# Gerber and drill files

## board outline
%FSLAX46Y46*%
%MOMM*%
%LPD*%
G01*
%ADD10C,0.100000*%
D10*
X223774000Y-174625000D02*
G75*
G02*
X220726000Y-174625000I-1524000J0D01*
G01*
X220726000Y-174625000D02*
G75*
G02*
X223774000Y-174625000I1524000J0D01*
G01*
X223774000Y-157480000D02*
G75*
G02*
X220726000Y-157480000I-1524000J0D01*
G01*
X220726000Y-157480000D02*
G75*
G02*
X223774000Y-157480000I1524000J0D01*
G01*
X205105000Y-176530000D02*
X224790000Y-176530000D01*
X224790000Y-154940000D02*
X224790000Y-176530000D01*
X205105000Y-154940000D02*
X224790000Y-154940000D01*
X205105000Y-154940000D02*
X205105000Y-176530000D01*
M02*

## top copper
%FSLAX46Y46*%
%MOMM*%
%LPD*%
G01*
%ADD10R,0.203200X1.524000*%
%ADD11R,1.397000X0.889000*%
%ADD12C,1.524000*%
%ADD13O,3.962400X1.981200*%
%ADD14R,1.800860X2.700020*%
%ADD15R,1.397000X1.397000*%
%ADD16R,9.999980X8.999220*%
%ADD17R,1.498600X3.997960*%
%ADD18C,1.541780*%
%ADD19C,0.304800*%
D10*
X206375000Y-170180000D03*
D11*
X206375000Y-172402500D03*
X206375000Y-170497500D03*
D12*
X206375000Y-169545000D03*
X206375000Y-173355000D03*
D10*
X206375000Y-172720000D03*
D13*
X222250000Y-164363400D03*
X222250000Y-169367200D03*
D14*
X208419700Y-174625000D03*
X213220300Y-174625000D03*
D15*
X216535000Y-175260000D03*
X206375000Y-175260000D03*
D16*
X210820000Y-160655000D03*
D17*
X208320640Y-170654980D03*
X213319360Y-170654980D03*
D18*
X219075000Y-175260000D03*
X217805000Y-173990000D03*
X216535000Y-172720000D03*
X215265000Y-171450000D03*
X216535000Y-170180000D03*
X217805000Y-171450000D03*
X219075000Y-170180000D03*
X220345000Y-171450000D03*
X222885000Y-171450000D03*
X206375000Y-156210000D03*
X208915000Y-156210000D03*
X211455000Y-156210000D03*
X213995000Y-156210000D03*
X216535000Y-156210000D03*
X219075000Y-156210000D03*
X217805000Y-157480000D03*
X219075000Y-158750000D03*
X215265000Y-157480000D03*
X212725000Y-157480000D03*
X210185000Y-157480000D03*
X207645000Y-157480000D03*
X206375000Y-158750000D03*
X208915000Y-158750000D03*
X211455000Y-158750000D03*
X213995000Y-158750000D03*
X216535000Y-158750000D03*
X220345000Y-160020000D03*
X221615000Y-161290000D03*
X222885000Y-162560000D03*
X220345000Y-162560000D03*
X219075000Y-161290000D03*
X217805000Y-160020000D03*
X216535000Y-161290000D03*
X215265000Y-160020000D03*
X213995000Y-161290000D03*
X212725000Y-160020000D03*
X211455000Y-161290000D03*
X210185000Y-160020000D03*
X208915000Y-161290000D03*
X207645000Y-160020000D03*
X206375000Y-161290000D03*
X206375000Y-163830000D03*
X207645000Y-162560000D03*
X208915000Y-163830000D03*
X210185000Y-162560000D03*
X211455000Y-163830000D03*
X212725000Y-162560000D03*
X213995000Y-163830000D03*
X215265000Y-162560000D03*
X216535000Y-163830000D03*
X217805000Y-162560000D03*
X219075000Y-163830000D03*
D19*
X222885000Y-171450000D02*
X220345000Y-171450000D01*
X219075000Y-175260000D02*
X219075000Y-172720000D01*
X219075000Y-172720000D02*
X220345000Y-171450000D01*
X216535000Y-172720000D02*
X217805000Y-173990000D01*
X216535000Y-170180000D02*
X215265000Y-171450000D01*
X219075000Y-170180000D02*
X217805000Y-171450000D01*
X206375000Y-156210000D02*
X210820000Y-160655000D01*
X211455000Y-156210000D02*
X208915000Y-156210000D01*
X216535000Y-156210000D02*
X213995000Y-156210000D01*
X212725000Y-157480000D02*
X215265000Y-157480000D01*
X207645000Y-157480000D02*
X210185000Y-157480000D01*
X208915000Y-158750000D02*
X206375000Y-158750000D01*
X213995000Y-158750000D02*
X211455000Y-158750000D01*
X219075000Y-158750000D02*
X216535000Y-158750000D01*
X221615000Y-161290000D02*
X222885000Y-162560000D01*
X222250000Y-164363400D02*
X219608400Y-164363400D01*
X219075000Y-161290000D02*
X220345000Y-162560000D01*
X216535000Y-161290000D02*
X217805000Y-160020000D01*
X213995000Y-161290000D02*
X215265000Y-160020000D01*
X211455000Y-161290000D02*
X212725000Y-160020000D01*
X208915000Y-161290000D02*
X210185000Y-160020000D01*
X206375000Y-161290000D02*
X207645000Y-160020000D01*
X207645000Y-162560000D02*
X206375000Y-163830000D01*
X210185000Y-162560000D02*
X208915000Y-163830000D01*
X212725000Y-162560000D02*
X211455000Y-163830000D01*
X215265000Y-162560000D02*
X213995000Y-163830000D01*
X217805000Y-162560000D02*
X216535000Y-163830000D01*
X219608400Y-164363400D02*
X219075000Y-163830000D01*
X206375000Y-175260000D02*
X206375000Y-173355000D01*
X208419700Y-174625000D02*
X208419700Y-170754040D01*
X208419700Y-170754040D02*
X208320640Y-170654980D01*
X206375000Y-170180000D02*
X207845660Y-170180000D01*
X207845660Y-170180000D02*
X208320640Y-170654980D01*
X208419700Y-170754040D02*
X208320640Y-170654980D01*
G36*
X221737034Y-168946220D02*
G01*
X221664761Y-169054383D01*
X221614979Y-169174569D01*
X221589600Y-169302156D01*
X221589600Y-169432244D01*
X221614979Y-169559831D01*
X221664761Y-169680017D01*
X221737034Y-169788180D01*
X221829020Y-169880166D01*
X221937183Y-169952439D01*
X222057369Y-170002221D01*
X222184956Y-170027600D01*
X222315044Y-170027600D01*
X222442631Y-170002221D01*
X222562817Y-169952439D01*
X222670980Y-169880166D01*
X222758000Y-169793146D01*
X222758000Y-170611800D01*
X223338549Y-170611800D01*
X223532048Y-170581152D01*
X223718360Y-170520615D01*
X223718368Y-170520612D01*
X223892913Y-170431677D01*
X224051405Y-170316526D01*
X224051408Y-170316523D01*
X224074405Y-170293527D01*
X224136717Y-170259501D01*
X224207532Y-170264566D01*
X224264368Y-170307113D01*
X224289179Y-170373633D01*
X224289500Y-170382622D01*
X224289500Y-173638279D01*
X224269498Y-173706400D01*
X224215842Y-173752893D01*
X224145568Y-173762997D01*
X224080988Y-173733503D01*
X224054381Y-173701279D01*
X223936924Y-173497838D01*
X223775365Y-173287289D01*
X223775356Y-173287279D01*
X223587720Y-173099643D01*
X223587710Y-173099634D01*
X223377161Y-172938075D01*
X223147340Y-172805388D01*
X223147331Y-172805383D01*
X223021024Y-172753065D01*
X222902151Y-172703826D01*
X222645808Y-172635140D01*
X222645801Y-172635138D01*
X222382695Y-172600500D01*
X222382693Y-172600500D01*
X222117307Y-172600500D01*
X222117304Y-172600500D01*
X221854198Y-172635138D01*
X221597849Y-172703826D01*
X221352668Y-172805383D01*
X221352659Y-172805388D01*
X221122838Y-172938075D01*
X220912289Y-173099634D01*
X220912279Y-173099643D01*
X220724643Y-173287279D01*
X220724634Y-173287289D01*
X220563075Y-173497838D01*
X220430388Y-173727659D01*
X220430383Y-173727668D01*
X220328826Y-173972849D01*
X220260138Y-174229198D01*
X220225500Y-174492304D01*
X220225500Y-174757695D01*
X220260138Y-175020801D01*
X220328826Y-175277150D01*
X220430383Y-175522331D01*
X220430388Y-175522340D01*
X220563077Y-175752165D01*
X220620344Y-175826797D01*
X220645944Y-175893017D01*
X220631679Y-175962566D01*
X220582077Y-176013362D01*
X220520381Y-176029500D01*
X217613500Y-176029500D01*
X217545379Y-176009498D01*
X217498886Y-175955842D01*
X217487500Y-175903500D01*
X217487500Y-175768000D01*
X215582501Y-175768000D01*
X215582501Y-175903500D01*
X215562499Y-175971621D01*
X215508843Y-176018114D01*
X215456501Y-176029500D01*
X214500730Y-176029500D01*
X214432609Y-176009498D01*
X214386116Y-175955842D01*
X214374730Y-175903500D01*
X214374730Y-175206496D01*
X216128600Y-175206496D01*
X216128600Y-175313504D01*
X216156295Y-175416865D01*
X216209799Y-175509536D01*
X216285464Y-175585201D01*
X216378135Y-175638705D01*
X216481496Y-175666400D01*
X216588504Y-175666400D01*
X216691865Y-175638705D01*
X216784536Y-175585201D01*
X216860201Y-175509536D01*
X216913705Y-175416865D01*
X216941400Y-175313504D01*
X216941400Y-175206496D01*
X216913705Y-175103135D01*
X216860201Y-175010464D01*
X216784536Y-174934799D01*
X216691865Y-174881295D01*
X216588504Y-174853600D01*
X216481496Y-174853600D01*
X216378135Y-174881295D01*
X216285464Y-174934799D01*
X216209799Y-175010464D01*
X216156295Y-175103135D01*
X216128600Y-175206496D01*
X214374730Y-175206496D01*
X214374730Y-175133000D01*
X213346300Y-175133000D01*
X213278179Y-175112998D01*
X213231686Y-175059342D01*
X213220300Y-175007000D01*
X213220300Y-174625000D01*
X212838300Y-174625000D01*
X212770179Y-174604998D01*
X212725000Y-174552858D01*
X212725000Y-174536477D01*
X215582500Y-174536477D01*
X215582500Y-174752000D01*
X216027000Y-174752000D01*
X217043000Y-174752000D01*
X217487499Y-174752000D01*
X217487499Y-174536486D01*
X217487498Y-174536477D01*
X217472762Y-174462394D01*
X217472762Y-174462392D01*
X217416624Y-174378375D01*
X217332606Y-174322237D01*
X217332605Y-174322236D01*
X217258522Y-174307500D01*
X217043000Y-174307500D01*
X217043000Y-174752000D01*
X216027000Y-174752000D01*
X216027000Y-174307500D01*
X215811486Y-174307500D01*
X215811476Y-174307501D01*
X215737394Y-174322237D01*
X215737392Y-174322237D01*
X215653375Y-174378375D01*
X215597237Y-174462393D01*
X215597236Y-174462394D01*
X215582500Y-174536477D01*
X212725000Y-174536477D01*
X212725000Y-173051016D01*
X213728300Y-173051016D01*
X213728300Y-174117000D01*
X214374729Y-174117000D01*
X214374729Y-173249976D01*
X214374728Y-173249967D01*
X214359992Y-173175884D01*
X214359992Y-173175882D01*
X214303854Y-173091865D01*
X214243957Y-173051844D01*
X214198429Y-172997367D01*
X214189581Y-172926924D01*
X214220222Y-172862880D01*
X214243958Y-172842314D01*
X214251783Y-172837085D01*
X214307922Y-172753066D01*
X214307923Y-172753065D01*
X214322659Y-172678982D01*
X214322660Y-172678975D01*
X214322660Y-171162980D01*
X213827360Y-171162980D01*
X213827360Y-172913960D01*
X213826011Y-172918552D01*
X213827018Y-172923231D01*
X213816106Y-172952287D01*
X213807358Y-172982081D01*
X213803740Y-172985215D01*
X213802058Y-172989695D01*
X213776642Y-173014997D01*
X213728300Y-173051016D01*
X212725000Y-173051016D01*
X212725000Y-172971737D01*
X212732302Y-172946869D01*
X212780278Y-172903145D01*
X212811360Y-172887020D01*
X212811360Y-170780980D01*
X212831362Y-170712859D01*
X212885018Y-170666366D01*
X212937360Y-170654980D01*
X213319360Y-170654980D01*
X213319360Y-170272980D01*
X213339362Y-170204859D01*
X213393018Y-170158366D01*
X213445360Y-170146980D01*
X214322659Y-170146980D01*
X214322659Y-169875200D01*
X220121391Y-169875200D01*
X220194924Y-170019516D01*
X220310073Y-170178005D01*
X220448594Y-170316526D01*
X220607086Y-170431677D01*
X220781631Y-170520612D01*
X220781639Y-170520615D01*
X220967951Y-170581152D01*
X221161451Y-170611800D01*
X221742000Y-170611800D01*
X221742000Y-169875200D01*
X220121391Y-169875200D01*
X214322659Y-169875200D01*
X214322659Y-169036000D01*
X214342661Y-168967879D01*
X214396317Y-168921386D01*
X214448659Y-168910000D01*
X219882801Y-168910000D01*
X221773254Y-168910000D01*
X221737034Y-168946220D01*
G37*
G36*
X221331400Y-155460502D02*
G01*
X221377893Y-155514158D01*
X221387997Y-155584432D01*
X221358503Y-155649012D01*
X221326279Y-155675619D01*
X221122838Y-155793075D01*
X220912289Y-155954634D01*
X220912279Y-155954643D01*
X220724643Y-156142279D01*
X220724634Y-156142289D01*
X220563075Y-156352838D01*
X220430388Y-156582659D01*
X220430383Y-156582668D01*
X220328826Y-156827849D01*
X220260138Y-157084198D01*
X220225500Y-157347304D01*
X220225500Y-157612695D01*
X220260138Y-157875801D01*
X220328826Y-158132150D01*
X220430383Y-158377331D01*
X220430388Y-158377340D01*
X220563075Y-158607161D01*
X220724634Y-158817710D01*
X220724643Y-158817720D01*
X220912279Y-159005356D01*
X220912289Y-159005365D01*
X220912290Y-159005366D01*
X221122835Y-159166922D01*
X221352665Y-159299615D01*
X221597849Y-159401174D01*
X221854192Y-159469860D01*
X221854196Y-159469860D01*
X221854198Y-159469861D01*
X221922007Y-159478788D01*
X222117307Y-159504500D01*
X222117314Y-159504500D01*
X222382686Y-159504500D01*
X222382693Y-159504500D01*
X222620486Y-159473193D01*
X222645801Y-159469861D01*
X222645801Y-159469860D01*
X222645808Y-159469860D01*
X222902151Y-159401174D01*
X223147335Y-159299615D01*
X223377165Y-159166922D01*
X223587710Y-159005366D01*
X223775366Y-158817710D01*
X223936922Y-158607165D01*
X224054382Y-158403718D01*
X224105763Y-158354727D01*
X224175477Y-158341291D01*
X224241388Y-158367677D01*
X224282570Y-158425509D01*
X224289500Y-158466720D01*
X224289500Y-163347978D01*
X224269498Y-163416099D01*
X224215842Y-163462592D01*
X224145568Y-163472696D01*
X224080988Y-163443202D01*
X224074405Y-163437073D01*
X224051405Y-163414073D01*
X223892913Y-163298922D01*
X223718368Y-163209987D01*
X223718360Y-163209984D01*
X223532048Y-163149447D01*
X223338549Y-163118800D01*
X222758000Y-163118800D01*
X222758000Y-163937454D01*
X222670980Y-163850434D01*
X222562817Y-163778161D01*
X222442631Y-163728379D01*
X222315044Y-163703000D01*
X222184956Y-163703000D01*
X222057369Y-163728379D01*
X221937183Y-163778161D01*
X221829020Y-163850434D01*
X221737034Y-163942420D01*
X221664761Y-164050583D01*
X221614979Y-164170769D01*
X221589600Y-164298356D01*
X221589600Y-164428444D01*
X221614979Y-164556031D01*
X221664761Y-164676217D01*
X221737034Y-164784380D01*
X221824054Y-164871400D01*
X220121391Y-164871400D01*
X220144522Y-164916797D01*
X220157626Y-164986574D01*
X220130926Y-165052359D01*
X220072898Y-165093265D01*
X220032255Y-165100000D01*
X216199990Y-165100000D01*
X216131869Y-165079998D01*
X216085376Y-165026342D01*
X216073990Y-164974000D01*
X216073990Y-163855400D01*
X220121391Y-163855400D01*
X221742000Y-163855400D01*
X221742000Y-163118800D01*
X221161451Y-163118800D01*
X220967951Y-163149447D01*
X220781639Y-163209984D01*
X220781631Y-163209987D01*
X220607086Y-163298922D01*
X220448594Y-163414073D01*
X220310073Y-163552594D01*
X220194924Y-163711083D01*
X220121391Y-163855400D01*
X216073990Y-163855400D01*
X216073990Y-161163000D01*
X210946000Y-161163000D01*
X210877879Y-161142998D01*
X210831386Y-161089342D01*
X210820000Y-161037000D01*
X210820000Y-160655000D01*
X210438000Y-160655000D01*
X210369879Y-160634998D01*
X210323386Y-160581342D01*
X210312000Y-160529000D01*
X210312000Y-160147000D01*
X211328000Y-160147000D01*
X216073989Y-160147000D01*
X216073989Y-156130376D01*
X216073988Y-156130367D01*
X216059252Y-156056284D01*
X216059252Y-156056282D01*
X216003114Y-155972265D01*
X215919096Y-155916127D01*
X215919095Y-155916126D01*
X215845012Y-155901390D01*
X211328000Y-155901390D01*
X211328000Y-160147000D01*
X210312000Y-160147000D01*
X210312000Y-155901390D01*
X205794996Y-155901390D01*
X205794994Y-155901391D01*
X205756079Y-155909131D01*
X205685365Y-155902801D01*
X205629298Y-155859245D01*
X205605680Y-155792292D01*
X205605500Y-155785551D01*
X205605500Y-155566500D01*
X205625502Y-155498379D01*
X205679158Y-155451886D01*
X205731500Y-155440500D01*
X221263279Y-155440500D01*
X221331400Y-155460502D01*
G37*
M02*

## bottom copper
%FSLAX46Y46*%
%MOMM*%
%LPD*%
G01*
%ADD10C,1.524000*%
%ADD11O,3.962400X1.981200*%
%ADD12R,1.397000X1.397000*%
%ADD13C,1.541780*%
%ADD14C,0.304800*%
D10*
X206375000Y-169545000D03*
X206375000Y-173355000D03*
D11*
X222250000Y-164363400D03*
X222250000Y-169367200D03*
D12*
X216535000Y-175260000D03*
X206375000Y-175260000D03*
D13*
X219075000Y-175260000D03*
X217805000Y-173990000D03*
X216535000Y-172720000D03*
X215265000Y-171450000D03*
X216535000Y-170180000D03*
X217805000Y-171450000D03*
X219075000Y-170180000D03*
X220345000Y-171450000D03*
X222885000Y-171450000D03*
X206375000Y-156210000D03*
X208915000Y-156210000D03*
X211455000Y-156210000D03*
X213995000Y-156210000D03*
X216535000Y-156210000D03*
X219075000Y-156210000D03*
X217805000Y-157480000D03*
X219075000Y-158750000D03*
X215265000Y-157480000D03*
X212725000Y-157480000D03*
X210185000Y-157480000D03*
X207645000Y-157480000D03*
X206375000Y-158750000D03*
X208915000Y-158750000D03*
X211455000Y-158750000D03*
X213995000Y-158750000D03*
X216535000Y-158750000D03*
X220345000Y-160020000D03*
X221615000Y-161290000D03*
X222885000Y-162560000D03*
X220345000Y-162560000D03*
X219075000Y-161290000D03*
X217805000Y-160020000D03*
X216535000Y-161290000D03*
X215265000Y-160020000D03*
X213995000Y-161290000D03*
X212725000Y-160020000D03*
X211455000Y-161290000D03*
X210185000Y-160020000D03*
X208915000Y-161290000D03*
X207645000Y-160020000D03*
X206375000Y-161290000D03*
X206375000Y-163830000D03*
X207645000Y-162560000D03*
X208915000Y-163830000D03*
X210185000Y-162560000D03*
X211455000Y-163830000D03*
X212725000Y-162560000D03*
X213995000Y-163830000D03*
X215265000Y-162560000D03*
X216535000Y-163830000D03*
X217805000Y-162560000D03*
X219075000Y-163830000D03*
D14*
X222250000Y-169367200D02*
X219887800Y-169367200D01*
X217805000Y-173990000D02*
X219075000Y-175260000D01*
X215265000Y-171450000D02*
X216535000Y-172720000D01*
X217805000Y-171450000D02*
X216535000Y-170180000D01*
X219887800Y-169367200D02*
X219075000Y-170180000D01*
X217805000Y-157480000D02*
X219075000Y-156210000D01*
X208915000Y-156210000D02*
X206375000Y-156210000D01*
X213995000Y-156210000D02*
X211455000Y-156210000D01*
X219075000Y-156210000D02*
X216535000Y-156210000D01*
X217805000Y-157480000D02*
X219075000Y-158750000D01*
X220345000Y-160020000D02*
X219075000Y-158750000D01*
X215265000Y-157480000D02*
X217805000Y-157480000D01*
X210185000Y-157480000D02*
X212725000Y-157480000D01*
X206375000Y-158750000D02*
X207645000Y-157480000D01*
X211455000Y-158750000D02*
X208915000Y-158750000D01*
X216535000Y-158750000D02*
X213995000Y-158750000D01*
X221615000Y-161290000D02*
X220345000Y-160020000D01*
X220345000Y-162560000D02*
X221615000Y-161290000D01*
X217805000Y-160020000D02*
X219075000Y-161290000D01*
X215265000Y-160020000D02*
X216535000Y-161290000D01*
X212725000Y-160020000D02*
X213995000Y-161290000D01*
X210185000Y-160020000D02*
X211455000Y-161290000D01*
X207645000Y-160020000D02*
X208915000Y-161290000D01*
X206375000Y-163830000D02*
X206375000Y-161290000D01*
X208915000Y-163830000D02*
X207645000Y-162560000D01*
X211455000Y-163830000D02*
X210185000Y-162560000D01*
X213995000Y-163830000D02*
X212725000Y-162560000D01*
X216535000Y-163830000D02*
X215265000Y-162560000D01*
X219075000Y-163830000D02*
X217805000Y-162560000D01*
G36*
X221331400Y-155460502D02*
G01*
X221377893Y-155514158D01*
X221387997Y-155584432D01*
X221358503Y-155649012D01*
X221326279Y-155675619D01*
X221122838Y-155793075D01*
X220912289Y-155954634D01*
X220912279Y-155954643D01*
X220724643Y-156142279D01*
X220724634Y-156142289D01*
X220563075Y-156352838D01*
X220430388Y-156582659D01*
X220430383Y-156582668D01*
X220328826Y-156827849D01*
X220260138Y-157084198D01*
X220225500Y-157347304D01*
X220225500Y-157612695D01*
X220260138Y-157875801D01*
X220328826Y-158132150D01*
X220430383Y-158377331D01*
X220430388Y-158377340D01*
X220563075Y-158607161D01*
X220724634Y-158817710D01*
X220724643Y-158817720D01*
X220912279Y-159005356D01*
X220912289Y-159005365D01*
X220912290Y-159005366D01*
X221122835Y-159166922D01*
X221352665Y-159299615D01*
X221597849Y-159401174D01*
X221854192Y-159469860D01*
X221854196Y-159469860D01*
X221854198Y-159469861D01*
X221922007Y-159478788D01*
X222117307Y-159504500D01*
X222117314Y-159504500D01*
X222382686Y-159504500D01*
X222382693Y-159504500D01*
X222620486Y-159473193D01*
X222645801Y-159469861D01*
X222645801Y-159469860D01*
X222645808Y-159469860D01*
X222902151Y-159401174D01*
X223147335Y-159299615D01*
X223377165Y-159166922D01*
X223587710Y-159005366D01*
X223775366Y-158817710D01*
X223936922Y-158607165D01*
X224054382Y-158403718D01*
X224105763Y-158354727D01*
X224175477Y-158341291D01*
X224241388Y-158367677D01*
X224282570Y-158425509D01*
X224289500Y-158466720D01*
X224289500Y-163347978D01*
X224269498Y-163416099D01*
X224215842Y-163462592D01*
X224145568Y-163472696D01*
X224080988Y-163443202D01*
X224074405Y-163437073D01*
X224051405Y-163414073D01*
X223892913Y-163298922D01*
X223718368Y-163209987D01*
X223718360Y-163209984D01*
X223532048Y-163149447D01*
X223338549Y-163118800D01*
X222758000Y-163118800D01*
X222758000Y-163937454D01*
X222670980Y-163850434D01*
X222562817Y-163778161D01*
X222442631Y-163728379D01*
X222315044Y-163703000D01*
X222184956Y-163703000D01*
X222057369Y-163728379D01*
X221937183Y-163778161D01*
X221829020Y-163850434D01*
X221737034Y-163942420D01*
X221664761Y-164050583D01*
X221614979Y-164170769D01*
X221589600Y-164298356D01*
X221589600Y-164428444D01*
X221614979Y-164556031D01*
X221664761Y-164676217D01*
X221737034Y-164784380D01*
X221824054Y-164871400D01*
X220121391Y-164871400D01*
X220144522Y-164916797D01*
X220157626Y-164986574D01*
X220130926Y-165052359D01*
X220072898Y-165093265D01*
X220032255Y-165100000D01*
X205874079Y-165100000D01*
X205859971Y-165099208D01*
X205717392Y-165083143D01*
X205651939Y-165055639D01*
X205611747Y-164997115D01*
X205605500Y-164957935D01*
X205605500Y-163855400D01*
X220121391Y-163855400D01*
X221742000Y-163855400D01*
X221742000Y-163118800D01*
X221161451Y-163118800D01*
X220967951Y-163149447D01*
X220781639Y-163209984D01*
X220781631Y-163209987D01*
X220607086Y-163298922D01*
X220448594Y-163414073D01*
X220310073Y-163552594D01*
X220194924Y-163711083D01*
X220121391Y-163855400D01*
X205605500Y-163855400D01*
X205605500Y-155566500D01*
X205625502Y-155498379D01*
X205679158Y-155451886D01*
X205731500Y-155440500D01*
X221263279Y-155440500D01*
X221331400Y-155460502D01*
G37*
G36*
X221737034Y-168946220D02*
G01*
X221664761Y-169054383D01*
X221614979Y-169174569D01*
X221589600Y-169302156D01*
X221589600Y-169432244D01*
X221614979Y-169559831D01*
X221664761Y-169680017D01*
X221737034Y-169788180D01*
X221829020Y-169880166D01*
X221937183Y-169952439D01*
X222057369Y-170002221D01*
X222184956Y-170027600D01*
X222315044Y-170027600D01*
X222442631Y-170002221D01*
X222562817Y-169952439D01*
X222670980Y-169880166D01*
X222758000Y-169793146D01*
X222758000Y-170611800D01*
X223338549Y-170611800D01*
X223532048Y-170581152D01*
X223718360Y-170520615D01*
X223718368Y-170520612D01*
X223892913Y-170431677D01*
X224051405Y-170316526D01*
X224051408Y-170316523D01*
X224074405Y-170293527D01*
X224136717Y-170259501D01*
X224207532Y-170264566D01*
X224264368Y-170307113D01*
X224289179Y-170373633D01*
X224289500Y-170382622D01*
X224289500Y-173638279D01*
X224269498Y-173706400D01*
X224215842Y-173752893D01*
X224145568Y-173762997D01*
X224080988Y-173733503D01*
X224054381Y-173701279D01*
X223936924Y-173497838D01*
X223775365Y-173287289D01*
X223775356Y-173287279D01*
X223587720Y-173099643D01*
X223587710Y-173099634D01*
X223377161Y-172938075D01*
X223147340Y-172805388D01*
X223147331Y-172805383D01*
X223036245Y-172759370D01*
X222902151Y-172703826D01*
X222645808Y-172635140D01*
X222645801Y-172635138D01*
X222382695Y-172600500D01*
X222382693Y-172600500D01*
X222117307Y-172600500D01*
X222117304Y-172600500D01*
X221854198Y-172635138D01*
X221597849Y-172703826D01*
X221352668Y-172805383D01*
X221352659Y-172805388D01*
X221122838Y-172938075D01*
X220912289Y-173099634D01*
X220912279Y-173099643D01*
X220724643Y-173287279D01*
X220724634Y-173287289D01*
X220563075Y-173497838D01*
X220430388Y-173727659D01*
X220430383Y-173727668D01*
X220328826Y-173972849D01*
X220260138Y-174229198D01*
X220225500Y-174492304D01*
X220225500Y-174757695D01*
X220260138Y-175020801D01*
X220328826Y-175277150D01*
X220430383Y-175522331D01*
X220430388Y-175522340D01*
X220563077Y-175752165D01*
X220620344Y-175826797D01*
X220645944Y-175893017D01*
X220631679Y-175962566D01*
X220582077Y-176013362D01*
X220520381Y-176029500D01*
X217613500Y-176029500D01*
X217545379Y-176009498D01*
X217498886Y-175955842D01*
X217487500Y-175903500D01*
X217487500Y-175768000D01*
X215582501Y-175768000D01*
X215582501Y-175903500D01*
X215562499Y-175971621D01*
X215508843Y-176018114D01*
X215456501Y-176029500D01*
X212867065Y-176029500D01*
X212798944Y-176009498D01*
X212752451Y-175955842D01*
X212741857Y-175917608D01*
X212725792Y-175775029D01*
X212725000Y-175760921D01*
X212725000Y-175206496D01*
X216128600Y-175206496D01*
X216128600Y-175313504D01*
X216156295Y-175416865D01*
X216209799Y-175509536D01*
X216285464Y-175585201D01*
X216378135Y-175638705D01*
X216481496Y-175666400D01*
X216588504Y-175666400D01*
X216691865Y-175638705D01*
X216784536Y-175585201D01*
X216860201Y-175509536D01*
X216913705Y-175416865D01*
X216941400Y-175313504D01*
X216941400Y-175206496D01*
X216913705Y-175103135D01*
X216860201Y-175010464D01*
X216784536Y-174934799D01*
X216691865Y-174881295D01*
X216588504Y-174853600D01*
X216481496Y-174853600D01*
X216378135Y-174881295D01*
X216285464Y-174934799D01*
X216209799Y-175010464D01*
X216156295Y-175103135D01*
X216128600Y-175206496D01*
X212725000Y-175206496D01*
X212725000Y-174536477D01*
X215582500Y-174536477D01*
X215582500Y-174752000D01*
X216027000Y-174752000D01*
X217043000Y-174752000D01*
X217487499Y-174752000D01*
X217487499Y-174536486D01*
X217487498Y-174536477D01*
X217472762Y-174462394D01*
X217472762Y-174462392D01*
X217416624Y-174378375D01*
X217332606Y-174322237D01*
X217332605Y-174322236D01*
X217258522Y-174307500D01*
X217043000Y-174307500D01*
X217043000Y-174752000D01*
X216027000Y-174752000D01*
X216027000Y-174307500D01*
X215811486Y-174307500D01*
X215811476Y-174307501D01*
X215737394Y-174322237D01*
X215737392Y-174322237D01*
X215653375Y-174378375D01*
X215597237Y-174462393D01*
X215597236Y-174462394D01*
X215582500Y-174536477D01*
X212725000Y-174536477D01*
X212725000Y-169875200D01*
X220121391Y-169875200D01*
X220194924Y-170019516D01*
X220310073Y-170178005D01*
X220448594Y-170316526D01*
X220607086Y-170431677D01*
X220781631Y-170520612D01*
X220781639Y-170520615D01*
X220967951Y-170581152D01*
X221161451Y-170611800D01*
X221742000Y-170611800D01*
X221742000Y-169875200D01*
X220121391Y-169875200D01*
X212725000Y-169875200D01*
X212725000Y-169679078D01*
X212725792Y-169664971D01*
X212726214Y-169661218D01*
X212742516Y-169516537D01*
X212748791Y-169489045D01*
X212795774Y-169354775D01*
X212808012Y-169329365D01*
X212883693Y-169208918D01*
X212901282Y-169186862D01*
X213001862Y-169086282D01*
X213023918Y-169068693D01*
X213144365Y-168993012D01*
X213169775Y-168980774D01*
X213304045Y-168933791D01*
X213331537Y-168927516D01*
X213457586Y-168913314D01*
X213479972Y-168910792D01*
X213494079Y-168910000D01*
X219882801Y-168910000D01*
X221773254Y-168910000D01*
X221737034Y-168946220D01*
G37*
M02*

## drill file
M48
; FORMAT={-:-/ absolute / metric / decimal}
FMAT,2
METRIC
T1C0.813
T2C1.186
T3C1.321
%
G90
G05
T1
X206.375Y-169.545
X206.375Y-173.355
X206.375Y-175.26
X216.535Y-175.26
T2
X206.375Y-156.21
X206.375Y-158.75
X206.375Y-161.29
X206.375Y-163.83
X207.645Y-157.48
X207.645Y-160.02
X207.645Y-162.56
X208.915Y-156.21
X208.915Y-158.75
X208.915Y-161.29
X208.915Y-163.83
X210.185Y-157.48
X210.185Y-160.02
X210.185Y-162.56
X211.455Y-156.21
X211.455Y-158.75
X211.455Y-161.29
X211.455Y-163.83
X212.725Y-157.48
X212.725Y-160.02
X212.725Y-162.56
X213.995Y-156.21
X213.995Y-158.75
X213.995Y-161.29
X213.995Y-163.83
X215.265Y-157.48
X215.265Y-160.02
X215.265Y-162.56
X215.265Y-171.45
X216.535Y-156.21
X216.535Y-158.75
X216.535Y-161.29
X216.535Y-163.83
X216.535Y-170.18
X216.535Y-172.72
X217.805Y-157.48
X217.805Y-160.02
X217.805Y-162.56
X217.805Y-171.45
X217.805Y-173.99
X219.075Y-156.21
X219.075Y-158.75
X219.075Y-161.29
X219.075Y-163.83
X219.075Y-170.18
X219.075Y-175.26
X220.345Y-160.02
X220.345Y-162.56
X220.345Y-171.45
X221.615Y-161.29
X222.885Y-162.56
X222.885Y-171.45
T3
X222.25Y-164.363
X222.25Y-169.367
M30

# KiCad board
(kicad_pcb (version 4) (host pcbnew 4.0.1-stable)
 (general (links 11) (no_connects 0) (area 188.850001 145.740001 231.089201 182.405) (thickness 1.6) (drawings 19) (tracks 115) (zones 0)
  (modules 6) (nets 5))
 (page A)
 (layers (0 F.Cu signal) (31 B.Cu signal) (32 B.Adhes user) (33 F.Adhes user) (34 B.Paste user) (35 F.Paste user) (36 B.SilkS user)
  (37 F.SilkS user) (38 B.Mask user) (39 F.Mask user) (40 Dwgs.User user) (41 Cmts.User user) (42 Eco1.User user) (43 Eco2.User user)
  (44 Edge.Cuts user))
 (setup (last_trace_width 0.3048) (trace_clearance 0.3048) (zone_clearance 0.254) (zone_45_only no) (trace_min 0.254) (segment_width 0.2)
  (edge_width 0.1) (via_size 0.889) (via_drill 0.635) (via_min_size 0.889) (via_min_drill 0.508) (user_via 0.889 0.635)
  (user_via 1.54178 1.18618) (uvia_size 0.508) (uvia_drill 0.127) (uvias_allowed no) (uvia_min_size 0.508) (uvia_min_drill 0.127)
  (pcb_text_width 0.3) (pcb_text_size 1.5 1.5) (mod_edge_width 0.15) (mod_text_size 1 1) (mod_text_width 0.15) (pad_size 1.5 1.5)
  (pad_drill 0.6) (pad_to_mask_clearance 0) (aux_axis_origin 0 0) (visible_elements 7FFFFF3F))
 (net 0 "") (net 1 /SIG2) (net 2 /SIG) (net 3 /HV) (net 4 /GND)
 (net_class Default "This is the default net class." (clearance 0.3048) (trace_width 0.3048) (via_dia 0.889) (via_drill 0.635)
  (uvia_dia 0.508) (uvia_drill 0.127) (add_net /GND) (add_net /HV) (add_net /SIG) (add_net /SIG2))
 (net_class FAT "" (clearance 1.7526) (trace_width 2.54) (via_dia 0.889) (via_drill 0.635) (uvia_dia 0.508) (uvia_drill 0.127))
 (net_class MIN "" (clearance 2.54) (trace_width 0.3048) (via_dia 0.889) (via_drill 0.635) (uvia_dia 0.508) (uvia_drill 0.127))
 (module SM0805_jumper (layer F.Cu) (at 206.375 171.45 90)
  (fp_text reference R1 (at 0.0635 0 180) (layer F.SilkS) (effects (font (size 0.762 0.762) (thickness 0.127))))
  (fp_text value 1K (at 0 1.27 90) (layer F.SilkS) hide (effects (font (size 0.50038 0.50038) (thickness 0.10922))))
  (pad 2 smd rect (at 1.27 0 90) (size 1.524 0.2032) (layers F.Cu F.Paste F.Mask) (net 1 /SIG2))
  (pad 1 smd rect (at -0.9525 0 90) (size 0.889 1.397) (layers F.Cu F.Paste F.Mask) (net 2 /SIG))
  (pad 2 smd rect (at 0.9525 0 90) (size 0.889 1.397) (layers F.Cu F.Paste F.Mask) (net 1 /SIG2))
  (pad 2 thru_hole circle (at 1.905 0 90) (size 1.524 1.524) (drill 0.8128) (layers *.Cu *.Mask F.SilkS) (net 1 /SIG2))
  (pad 1 thru_hole circle (at -1.905 0 90) (size 1.524 1.524) (drill 0.8128) (layers *.Cu *.Mask F.SilkS) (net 2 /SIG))
  (pad 1 smd rect (at -1.27 0 90) (size 1.524 0.2032) (layers F.Cu F.Paste F.Mask) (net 2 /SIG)))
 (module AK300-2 (layer F.Cu) (at 222.25 166.878 270)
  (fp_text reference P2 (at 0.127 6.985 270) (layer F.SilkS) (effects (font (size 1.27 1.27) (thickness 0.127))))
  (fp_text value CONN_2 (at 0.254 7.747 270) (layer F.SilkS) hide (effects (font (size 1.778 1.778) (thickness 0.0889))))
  (pad 1 thru_hole oval (at -2.5146 0 270) (size 1.9812 3.9624) (drill 1.3208) (layers *.Cu F.Paste F.SilkS F.Mask) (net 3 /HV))
  (pad 2 thru_hole oval (at 2.4892 0 270) (size 1.9812 3.9624) (drill 1.3208) (layers *.Cu F.Paste F.SilkS F.Mask) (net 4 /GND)))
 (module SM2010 (layer F.Cu) (at 210.82 174.625)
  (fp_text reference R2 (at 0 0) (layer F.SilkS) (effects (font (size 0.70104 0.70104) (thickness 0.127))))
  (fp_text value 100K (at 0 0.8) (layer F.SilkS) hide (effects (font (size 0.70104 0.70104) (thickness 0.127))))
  (pad 1 smd rect (at -2.4003 0) (size 1.80086 2.70002) (layers F.Cu F.Paste F.Mask) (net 1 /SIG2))
  (pad 2 smd rect (at 2.4003 0) (size 1.80086 2.70002) (layers F.Cu F.Paste F.Mask) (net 4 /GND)))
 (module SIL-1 (layer F.Cu) (at 216.535 175.26)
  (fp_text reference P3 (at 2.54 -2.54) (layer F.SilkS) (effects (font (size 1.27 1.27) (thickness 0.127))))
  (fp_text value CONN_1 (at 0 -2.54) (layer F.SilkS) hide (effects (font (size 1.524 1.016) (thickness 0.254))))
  (pad 1 thru_hole rect (at 0 0) (size 1.397 1.397) (drill 0.8128) (layers *.Cu *.Mask F.SilkS) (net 4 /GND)))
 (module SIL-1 (layer F.Cu) (at 206.375 175.26 180)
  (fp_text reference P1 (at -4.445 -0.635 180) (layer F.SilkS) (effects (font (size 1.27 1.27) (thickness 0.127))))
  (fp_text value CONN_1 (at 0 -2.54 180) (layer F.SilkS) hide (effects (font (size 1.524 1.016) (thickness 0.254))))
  (pad 1 thru_hole rect (at 0 0 180) (size 1.397 1.397) (drill 0.8128) (layers *.Cu *.Mask F.SilkS) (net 2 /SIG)))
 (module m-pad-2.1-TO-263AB (layer F.Cu) (at 210.82 160.655)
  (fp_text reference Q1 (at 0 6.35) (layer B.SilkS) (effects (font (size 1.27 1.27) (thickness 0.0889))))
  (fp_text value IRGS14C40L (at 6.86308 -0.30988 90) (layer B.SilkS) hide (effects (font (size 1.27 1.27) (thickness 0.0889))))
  (pad 2 smd rect (at 0 0) (size 9.99998 8.99922) (layers F.Cu F.Paste F.Mask) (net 3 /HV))
  (pad 1 smd rect (at -2.49936 9.99998) (size 1.4986 3.99796) (layers F.Cu F.Paste F.Mask) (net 1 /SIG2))
  (pad 3 smd rect (at 2.49936 9.99998) (size 1.4986 3.99796) (layers F.Cu F.Paste F.Mask) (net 4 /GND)))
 (gr_circle (center 222.25 174.625) (end 223.774 174.625) (layer Edge.Cuts) (width 0.1))
 (gr_circle (center 222.25 157.48) (end 223.774 157.48) (layer Edge.Cuts) (width 0.1))
 (gr_line (start 205.105 176.53) (end 224.79 176.53) (angle 90) (layer Edge.Cuts) (width 0.1))
 (gr_line (start 224.79 154.94) (end 224.79 176.53) (angle 90) (layer Edge.Cuts) (width 0.1))
 (gr_line (start 205.105 154.94) (end 224.79 154.94) (angle 90) (layer Edge.Cuts) (width 0.1))
 (gr_line (start 205.105 154.94) (end 205.105 176.53) (angle 90) (layer Edge.Cuts) (width 0.1))
 (segment (start 222.885 171.45) (end 220.345 171.45) (width 0.3048) (layer F.Cu) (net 4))
 (segment (start 219.075 175.26) (end 219.075 172.72) (width 0.3048) (layer F.Cu) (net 4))
 (segment (start 222.25 169.3672) (end 219.8878 169.3672) (width 0.3048) (layer B.Cu) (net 4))
 (segment (start 219.075 172.72) (end 220.345 171.45) (width 0.3048) (layer F.Cu) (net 4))
 (via (at 219.075 175.26) (size 1.54178) (drill 1.18618) (layers F.Cu B.Cu) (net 4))
 (segment (start 217.805 173.99) (end 219.075 175.26) (width 0.3048) (layer B.Cu) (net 4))
 (via (at 217.805 173.99) (size 1.54178) (drill 1.18618) (layers F.Cu B.Cu) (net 4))
 (segment (start 216.535 172.72) (end 217.805 173.99) (width 0.3048) (layer F.Cu) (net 4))
 (via (at 216.535 172.72) (size 1.54178) (drill 1.18618) (layers F.Cu B.Cu) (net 4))
 (segment (start 215.265 171.45) (end 216.535 172.72) (width 0.3048) (layer B.Cu) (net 4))
 (via (at 215.265 171.45) (size 1.54178) (drill 1.18618) (layers F.Cu B.Cu) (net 4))
 (segment (start 216.535 170.18) (end 215.265 171.45) (width 0.3048) (layer F.Cu) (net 4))
 (via (at 216.535 170.18) (size 1.54178) (drill 1.18618) (layers F.Cu B.Cu) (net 4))
 (segment (start 217.805 171.45) (end 216.535 170.18) (width 0.3048) (layer B.Cu) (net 4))
 (via (at 217.805 171.45) (size 1.54178) (drill 1.18618) (layers F.Cu B.Cu) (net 4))
 (segment (start 219.075 170.18) (end 217.805 171.45) (width 0.3048) (layer F.Cu) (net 4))
 (via (at 219.075 170.18) (size 1.54178) (drill 1.18618) (layers F.Cu B.Cu) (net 4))
 (segment (start 219.8878 169.3672) (end 219.075 170.18) (width 0.3048) (layer B.Cu) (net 4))
 (via (at 220.345 171.45) (size 1.54178) (drill 1.18618) (layers F.Cu B.Cu) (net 4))
 (via (at 222.885 171.45) (size 1.54178) (drill 1.18618) (layers F.Cu B.Cu) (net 4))
 (segment (start 217.805 157.48) (end 219.075 156.21) (width 0.3048) (layer B.Cu) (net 3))
 (segment (start 206.375 156.21) (end 210.82 160.655) (width 0.3048) (layer F.Cu) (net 3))
 (via (at 206.375 156.21) (size 1.54178) (drill 1.18618) (layers F.Cu B.Cu) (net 3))
 (segment (start 208.915 156.21) (end 206.375 156.21) (width 0.3048) (layer B.Cu) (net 3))
 (via (at 208.915 156.21) (size 1.54178) (drill 1.18618) (layers F.Cu B.Cu) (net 3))
 (segment (start 211.455 156.21) (end 208.915 156.21) (width 0.3048) (layer F.Cu) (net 3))
 (via (at 211.455 156.21) (size 1.54178) (drill 1.18618) (layers F.Cu B.Cu) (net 3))
 (segment (start 213.995 156.21) (end 211.455 156.21) (width 0.3048) (layer B.Cu) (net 3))
 (via (at 213.995 156.21) (size 1.54178) (drill 1.18618) (layers F.Cu B.Cu) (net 3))
 (segment (start 216.535 156.21) (end 213.995 156.21) (width 0.3048) (layer F.Cu) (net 3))
 (via (at 216.535 156.21) (size 1.54178) (drill 1.18618) (layers F.Cu B.Cu) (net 3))
 (segment (start 219.075 156.21) (end 216.535 156.21) (width 0.3048) (layer B.Cu) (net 3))
 (via (at 219.075 156.21) (size 1.54178) (drill 1.18618) (layers F.Cu B.Cu) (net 3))
 (via (at 217.805 157.48) (size 1.54178) (drill 1.18618) (layers F.Cu B.Cu) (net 3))
 (segment (start 217.805 157.48) (end 219.075 158.75) (width 0.3048) (layer B.Cu) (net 3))
 (segment (start 220.345 160.02) (end 219.075 158.75) (width 0.3048) (layer B.Cu) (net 3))
 (via (at 219.075 158.75) (size 1.54178) (drill 1.18618) (layers F.Cu B.Cu) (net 3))
 (segment (start 215.265 157.48) (end 217.805 157.48) (width 0.3048) (layer B.Cu) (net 3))
 (via (at 215.265 157.48) (size 1.54178) (drill 1.18618) (layers F.Cu B.Cu) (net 3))
 (segment (start 212.725 157.48) (end 215.265 157.48) (width 0.3048) (layer F.Cu) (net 3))
 (via (at 212.725 157.48) (size 1.54178) (drill 1.18618) (layers F.Cu B.Cu) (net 3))
 (segment (start 210.185 157.48) (end 212.725 157.48) (width 0.3048) (layer B.Cu) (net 3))
 (via (at 210.185 157.48) (size 1.54178) (drill 1.18618) (layers F.Cu B.Cu) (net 3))
 (segment (start 207.645 157.48) (end 210.185 157.48) (width 0.3048) (layer F.Cu) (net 3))
 (via (at 207.645 157.48) (size 1.54178) (drill 1.18618) (layers F.Cu B.Cu) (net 3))
 (segment (start 206.375 158.75) (end 207.645 157.48) (width 0.3048) (layer B.Cu) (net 3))
 (via (at 206.375 158.75) (size 1.54178) (drill 1.18618) (layers F.Cu B.Cu) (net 3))
 (segment (start 208.915 158.75) (end 206.375 158.75) (width 0.3048) (layer F.Cu) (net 3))
 (via (at 208.915 158.75) (size 1.54178) (drill 1.18618) (layers F.Cu B.Cu) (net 3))
 (segment (start 211.455 158.75) (end 208.915 158.75) (width 0.3048) (layer B.Cu) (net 3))
 (via (at 211.455 158.75) (size 1.54178) (drill 1.18618) (layers F.Cu B.Cu) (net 3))
 (segment (start 213.995 158.75) (end 211.455 158.75) (width 0.3048) (layer F.Cu) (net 3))
 (via (at 213.995 158.75) (size 1.54178) (drill 1.18618) (layers F.Cu B.Cu) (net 3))
 (segment (start 216.535 158.75) (end 213.995 158.75) (width 0.3048) (layer B.Cu) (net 3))
 (via (at 216.535 158.75) (size 1.54178) (drill 1.18618) (layers F.Cu B.Cu) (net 3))
 (segment (start 219.075 158.75) (end 216.535 158.75) (width 0.3048) (layer F.Cu) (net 3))
 (via (at 220.345 160.02) (size 1.54178) (drill 1.18618) (layers F.Cu B.Cu) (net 3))
 (segment (start 221.615 161.29) (end 220.345 160.02) (width 0.3048) (layer B.Cu) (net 3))
 (via (at 221.615 161.29) (size 1.54178) (drill 1.18618) (layers F.Cu B.Cu) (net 3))
 (via (at 222.885 162.56) (size 1.54178) (drill 1.18618) (layers F.Cu B.Cu) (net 3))
 (segment (start 221.615 161.29) (end 222.885 162.56) (width 0.3048) (layer F.Cu) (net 3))
 (segment (start 222.25 164.3634) (end 219.6084 164.3634) (width 0.3048) (layer F.Cu) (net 3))
 (segment (start 220.345 162.56) (end 221.615 161.29) (width 0.3048) (layer B.Cu) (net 3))
 (via (at 220.345 162.56) (size 1.54178) (drill 1.18618) (layers F.Cu B.Cu) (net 3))
 (segment (start 219.075 161.29) (end 220.345 162.56) (width 0.3048) (layer F.Cu) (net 3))
 (via (at 219.075 161.29) (size 1.54178) (drill 1.18618) (layers F.Cu B.Cu) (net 3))
 (segment (start 217.805 160.02) (end 219.075 161.29) (width 0.3048) (layer B.Cu) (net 3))
 (via (at 217.805 160.02) (size 1.54178) (drill 1.18618) (layers F.Cu B.Cu) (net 3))
 (segment (start 216.535 161.29) (end 217.805 160.02) (width 0.3048) (layer F.Cu) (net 3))
 (via (at 216.535 161.29) (size 1.54178) (drill 1.18618) (layers F.Cu B.Cu) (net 3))
 (segment (start 215.265 160.02) (end 216.535 161.29) (width 0.3048) (layer B.Cu) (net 3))
 (via (at 215.265 160.02) (size 1.54178) (drill 1.18618) (layers F.Cu B.Cu) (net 3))
 (segment (start 213.995 161.29) (end 215.265 160.02) (width 0.3048) (layer F.Cu) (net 3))
 (via (at 213.995 161.29) (size 1.54178) (drill 1.18618) (layers F.Cu B.Cu) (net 3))
 (segment (start 212.725 160.02) (end 213.995 161.29) (width 0.3048) (layer B.Cu) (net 3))
 (via (at 212.725 160.02) (size 1.54178) (drill 1.18618) (layers F.Cu B.Cu) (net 3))
 (segment (start 211.455 161.29) (end 212.725 160.02) (width 0.3048) (layer F.Cu) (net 3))
 (via (at 211.455 161.29) (size 1.54178) (drill 1.18618) (layers F.Cu B.Cu) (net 3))
 (segment (start 210.185 160.02) (end 211.455 161.29) (width 0.3048) (layer B.Cu) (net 3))
 (via (at 210.185 160.02) (size 1.54178) (drill 1.18618) (layers F.Cu B.Cu) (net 3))
 (segment (start 208.915 161.29) (end 210.185 160.02) (width 0.3048) (layer F.Cu) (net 3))
 (via (at 208.915 161.29) (size 1.54178) (drill 1.18618) (layers F.Cu B.Cu) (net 3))
 (segment (start 207.645 160.02) (end 208.915 161.29) (width 0.3048) (layer B.Cu) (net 3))
 (via (at 207.645 160.02) (size 1.54178) (drill 1.18618) (layers F.Cu B.Cu) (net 3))
 (segment (start 206.375 161.29) (end 207.645 160.02) (width 0.3048) (layer F.Cu) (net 3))
 (via (at 206.375 161.29) (size 1.54178) (drill 1.18618) (layers F.Cu B.Cu) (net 3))
 (segment (start 206.375 163.83) (end 206.375 161.29) (width 0.3048) (layer B.Cu) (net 3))
 (via (at 206.375 163.83) (size 1.54178) (drill 1.18618) (layers F.Cu B.Cu) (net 3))
 (segment (start 207.645 162.56) (end 206.375 163.83) (width 0.3048) (layer F.Cu) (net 3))
 (via (at 207.645 162.56) (size 1.54178) (drill 1.18618) (layers F.Cu B.Cu) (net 3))
 (segment (start 208.915 163.83) (end 207.645 162.56) (width 0.3048) (layer B.Cu) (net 3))
 (via (at 208.915 163.83) (size 1.54178) (drill 1.18618) (layers F.Cu B.Cu) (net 3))
 (segment (start 210.185 162.56) (end 208.915 163.83) (width 0.3048) (layer F.Cu) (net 3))
 (via (at 210.185 162.56) (size 1.54178) (drill 1.18618) (layers F.Cu B.Cu) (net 3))
 (segment (start 211.455 163.83) (end 210.185 162.56) (width 0.3048) (layer B.Cu) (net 3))
 (via (at 211.455 163.83) (size 1.54178) (drill 1.18618) (layers F.Cu B.Cu) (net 3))
 (segment (start 212.725 162.56) (end 211.455 163.83) (width 0.3048) (layer F.Cu) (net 3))
 (via (at 212.725 162.56) (size 1.54178) (drill 1.18618) (layers F.Cu B.Cu) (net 3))
 (segment (start 213.995 163.83) (end 212.725 162.56) (width 0.3048) (layer B.Cu) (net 3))
 (via (at 213.995 163.83) (size 1.54178) (drill 1.18618) (layers F.Cu B.Cu) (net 3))
 (segment (start 215.265 162.56) (end 213.995 163.83) (width 0.3048) (layer F.Cu) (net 3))
 (via (at 215.265 162.56) (size 1.54178) (drill 1.18618) (layers F.Cu B.Cu) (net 3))
 (segment (start 216.535 163.83) (end 215.265 162.56) (width 0.3048) (layer B.Cu) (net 3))
 (via (at 216.535 163.83) (size 1.54178) (drill 1.18618) (layers F.Cu B.Cu) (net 3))
 (segment (start 217.805 162.56) (end 216.535 163.83) (width 0.3048) (layer F.Cu) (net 3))
 (via (at 217.805 162.56) (size 1.54178) (drill 1.18618) (layers F.Cu B.Cu) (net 3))
 (segment (start 219.075 163.83) (end 217.805 162.56) (width 0.3048) (layer B.Cu) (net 3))
 (via (at 219.075 163.83) (size 1.54178) (drill 1.18618) (layers F.Cu B.Cu) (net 3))
 (segment (start 219.6084 164.3634) (end 219.075 163.83) (width 0.3048) (layer F.Cu) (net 3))
 (segment (start 206.375 175.26) (end 206.375 173.355) (width 0.3048) (layer F.Cu) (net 2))
 (segment (start 208.4197 174.625) (end 208.4197 170.75404) (width 0.3048) (layer F.Cu) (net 1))
 (segment (start 208.4197 170.75404) (end 208.32064 170.65498) (width 0.3048) (layer F.Cu) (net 1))
 (segment (start 206.375 170.18) (end 207.84566 170.18) (width 0.3048) (layer F.Cu) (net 1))
 (segment (start 207.84566 170.18) (end 208.32064 170.65498) (width 0.3048) (layer F.Cu) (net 1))
 (segment (start 208.4197 170.75404) (end 208.32064 170.65498) (width 0.3048) (layer F.Cu) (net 1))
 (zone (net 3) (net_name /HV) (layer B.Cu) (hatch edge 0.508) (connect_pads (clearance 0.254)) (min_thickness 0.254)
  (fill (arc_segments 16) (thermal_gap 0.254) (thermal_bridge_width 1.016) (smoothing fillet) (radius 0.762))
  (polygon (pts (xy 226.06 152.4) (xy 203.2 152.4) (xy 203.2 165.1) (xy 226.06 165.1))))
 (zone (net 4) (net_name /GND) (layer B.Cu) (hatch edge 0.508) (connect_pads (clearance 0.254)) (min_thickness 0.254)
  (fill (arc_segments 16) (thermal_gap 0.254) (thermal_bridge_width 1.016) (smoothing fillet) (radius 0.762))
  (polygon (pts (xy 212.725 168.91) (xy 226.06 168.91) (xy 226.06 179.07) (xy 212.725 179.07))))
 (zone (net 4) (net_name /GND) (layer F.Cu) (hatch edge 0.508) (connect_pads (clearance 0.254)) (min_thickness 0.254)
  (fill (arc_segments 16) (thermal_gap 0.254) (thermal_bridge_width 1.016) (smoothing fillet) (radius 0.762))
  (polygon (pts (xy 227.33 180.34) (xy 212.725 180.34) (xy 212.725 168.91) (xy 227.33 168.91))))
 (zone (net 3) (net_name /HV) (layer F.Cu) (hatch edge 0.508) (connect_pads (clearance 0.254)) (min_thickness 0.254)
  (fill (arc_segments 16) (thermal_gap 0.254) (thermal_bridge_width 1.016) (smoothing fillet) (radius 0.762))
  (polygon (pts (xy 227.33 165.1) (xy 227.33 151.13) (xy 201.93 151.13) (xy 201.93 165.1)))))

